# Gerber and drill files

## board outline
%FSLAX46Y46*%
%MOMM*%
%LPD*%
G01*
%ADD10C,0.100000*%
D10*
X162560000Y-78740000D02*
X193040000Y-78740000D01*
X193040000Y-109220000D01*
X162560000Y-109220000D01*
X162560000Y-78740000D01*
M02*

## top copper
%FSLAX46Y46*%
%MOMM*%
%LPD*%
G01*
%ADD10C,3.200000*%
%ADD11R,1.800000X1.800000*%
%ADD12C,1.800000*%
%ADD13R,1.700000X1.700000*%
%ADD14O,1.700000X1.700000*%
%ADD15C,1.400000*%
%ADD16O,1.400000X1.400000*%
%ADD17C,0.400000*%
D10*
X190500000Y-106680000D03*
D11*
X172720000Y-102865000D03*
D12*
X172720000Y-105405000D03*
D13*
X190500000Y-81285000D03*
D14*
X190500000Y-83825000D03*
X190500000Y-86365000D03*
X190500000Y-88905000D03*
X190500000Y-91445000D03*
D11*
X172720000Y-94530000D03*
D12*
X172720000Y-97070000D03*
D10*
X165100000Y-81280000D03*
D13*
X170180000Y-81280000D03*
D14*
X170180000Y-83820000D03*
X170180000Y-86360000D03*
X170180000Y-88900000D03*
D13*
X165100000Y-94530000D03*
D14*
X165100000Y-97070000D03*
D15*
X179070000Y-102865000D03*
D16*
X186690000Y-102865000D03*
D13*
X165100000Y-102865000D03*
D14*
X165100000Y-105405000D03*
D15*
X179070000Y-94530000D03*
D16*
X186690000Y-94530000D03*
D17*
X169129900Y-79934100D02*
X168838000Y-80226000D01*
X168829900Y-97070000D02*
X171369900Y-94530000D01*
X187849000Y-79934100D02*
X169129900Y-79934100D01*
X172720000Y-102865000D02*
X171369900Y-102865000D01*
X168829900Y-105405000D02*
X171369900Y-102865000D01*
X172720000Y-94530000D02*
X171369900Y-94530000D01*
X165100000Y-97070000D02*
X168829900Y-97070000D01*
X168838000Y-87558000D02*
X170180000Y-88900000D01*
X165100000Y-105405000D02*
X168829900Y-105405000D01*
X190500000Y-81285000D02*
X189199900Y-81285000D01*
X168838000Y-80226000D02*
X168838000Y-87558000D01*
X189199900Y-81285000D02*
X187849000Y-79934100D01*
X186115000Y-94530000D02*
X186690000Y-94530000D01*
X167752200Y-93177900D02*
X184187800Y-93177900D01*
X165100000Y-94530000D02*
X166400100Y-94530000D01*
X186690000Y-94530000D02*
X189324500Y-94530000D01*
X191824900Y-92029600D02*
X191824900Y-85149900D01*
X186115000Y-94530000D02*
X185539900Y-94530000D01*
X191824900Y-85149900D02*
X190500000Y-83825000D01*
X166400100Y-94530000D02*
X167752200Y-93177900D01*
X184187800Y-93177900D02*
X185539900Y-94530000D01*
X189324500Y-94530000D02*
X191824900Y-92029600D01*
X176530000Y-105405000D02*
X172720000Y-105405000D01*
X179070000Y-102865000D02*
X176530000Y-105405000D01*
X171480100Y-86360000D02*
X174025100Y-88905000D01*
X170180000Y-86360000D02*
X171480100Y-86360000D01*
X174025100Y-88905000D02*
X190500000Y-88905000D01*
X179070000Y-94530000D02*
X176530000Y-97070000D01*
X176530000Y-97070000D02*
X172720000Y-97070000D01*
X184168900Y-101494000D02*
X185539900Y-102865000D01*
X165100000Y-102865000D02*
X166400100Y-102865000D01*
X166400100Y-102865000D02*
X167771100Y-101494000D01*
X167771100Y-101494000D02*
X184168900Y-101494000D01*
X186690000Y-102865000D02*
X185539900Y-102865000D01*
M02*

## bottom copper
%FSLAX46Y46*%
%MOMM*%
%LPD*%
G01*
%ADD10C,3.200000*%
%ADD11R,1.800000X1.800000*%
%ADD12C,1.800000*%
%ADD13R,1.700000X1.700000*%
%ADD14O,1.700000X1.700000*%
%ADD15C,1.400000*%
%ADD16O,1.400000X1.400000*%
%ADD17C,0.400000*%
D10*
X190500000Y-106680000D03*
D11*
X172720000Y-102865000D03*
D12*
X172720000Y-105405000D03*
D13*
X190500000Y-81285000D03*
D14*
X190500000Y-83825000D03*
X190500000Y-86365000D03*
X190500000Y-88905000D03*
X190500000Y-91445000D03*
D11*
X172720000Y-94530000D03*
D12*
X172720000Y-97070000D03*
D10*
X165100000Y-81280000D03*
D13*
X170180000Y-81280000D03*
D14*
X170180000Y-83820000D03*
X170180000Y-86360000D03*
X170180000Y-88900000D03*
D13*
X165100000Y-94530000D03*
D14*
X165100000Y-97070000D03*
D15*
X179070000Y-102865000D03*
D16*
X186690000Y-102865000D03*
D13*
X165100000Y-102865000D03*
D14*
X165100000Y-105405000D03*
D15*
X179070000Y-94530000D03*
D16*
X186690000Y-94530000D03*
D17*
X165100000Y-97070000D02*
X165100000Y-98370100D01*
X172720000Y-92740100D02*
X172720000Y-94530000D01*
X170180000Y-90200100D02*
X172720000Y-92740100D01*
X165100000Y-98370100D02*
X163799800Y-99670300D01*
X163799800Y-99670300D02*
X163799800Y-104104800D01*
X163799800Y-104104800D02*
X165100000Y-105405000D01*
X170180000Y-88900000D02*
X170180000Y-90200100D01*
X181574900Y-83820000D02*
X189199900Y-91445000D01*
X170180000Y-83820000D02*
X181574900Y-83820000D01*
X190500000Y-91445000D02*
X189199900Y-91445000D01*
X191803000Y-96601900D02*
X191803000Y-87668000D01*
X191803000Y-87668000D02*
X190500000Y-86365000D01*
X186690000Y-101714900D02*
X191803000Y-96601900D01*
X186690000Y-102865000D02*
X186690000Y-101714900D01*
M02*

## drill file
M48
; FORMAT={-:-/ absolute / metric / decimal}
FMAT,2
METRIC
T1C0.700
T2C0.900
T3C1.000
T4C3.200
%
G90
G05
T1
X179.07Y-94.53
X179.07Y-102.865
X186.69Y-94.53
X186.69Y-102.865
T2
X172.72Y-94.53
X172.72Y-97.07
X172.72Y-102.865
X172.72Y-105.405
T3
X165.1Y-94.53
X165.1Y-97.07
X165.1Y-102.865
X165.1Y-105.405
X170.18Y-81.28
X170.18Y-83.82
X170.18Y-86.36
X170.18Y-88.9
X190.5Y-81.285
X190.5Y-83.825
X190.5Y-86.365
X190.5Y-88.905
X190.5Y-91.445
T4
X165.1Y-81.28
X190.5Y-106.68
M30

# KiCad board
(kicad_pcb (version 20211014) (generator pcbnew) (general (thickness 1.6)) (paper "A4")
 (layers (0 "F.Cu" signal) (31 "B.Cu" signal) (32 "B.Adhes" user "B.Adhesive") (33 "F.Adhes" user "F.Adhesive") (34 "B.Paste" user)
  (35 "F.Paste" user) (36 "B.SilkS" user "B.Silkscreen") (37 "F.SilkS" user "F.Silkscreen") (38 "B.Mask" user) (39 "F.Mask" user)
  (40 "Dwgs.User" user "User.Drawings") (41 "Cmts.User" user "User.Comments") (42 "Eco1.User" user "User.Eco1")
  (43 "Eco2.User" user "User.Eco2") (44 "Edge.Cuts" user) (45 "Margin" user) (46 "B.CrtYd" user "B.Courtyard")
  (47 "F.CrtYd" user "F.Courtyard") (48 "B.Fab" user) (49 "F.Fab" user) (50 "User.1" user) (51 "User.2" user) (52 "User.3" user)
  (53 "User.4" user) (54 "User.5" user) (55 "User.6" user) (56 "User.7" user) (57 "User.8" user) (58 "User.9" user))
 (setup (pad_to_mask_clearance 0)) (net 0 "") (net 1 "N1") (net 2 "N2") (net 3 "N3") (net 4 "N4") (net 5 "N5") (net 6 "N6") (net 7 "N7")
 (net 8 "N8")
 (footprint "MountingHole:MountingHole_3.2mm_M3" (layer "F.Cu") (at 190.5 106.68)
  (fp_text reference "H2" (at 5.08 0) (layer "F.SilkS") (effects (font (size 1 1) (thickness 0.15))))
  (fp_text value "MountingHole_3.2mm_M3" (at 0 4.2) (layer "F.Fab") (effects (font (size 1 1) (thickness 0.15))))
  (pad "" thru_hole circle (at 0 0) (size 3.2 3.2) (drill 3.2) (layers *.Cu *.Mask)))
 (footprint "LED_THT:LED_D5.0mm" (layer "F.Cu") (at 172.72 102.865 -90)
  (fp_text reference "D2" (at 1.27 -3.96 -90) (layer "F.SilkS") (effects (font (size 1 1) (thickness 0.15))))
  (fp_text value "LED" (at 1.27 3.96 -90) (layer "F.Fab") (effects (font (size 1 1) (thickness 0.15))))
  (pad "1" thru_hole rect (at 0 0 270) (size 1.8 1.8) (drill 0.9) (layers *.Cu *.Mask) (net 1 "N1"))
  (pad "2" thru_hole circle (at 2.54 0 270) (size 1.8 1.8) (drill 0.9) (layers *.Cu *.Mask) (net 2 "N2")))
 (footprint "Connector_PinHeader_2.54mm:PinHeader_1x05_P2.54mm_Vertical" (layer "F.Cu") (at 190.5 81.285)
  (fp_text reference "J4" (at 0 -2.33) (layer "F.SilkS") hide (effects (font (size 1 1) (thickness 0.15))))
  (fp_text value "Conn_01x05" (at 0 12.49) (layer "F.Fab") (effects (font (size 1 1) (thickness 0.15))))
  (pad "1" thru_hole rect (at 0 0) (size 1.7 1.7) (drill 1) (layers *.Cu *.Mask) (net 1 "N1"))
  (pad "2" thru_hole oval (at 0 2.54) (size 1.7 1.7) (drill 1) (layers *.Cu *.Mask) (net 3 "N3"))
  (pad "3" thru_hole oval (at 0 5.08) (size 1.7 1.7) (drill 1) (layers *.Cu *.Mask) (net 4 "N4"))
  (pad "4" thru_hole oval (at 0 7.62) (size 1.7 1.7) (drill 1) (layers *.Cu *.Mask) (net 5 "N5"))
  (pad "5" thru_hole oval (at 0 10.16) (size 1.7 1.7) (drill 1) (layers *.Cu *.Mask) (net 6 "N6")))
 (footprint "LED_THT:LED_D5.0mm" (layer "F.Cu") (at 172.72 94.53 -90)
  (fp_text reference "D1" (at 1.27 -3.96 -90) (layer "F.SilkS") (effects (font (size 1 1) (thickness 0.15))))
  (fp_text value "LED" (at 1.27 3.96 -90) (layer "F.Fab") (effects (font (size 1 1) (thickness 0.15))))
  (pad "1" thru_hole rect (at 0 0 270) (size 1.8 1.8) (drill 0.9) (layers *.Cu *.Mask) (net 1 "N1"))
  (pad "2" thru_hole circle (at 2.54 0 270) (size 1.8 1.8) (drill 0.9) (layers *.Cu *.Mask) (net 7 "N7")))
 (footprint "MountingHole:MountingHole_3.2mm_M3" (layer "F.Cu") (at 165.1 81.28)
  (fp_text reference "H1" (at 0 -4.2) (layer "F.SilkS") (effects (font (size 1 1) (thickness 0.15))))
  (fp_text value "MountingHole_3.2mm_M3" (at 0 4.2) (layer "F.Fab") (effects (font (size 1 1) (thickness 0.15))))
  (pad "" thru_hole circle (at 0 0) (size 3.2 3.2) (drill 3.2) (layers *.Cu *.Mask)))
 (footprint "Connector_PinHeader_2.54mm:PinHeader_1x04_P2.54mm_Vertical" (layer "F.Cu") (at 170.18 81.28)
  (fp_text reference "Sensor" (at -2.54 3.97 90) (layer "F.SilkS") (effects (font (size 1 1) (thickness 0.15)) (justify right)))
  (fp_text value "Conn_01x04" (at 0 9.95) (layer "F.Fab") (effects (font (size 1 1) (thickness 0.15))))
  (pad "1" thru_hole rect (at 0 0) (size 1.7 1.7) (drill 1) (layers *.Cu *.Mask) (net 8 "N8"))
  (pad "2" thru_hole oval (at 0 2.54) (size 1.7 1.7) (drill 1) (layers *.Cu *.Mask) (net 6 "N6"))
  (pad "3" thru_hole oval (at 0 5.08) (size 1.7 1.7) (drill 1) (layers *.Cu *.Mask) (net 5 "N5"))
  (pad "4" thru_hole oval (at 0 7.62) (size 1.7 1.7) (drill 1) (layers *.Cu *.Mask) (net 1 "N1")))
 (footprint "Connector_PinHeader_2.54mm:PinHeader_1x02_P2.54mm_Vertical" (layer "F.Cu") (at 165.1 94.53)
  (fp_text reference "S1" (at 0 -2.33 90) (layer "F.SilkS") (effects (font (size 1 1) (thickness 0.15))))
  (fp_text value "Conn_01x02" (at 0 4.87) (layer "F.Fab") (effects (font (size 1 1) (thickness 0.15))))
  (pad "1" thru_hole rect (at 0 0) (size 1.7 1.7) (drill 1) (layers *.Cu *.Mask) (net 3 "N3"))
  (pad "2" thru_hole oval (at 0 2.54) (size 1.7 1.7) (drill 1) (layers *.Cu *.Mask) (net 1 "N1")))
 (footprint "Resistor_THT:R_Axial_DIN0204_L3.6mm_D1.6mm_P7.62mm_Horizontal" (layer "F.Cu") (at 179.07 102.865)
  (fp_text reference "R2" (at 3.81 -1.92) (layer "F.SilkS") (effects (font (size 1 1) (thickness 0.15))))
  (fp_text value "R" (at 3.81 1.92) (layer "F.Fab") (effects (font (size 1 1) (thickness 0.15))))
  (pad "1" thru_hole circle (at 0 0) (size 1.4 1.4) (drill 0.7) (layers *.Cu *.Mask) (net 2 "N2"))
  (pad "2" thru_hole oval (at 7.62 0) (size 1.4 1.4) (drill 0.7) (layers *.Cu *.Mask) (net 4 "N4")))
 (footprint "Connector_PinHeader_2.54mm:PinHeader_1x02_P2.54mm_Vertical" (layer "F.Cu") (at 165.1 102.865)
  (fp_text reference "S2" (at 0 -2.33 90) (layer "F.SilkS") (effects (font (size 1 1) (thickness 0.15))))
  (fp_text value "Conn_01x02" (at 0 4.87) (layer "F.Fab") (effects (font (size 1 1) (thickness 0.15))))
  (pad "1" thru_hole rect (at 0 0) (size 1.7 1.7) (drill 1) (layers *.Cu *.Mask) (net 4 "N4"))
  (pad "2" thru_hole oval (at 0 2.54) (size 1.7 1.7) (drill 1) (layers *.Cu *.Mask) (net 1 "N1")))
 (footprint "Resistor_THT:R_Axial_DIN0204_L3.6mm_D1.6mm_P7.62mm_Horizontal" (layer "F.Cu") (at 179.07 94.53)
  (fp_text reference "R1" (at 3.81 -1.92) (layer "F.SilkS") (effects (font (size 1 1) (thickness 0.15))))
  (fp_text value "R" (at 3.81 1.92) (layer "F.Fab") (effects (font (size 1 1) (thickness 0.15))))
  (pad "1" thru_hole circle (at 0 0) (size 1.4 1.4) (drill 0.7) (layers *.Cu *.Mask) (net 7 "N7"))
  (pad "2" thru_hole oval (at 7.62 0) (size 1.4 1.4) (drill 0.7) (layers *.Cu *.Mask) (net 3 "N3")))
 (gr_rect (start 162.56 78.74) (end 193.04 109.22) (layer "Edge.Cuts") (width 0.1) (fill none))
 (segment (start 169.1299 79.9341) (end 168.838 80.226) (width 0.4) (layer "F.Cu") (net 1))
 (segment (start 168.8299 97.07) (end 171.3699 94.53) (width 0.4) (layer "F.Cu") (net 1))
 (segment (start 187.849 79.9341) (end 169.1299 79.9341) (width 0.4) (layer "F.Cu") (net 1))
 (segment (start 172.72 102.865) (end 171.3699 102.865) (width 0.4) (layer "F.Cu") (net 1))
 (segment (start 168.8299 105.405) (end 171.3699 102.865) (width 0.4) (layer "F.Cu") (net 1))
 (segment (start 172.72 94.53) (end 171.3699 94.53) (width 0.4) (layer "F.Cu") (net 1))
 (segment (start 165.1 97.07) (end 168.8299 97.07) (width 0.4) (layer "F.Cu") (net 1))
 (segment (start 168.838 87.558) (end 170.18 88.9) (width 0.4) (layer "F.Cu") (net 1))
 (segment (start 165.1 105.405) (end 168.8299 105.405) (width 0.4) (layer "F.Cu") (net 1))
 (segment (start 190.5 81.285) (end 189.1999 81.285) (width 0.4) (layer "F.Cu") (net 1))
 (segment (start 168.838 80.226) (end 168.838 87.558) (width 0.4) (layer "F.Cu") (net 1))
 (segment (start 189.1999 81.285) (end 187.849 79.9341) (width 0.4) (layer "F.Cu") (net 1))
 (segment (start 165.1 97.07) (end 165.1 98.3701) (width 0.4) (layer "B.Cu") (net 1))
 (segment (start 172.72 92.7401) (end 172.72 94.53) (width 0.4) (layer "B.Cu") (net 1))
 (segment (start 170.18 90.2001) (end 172.72 92.7401) (width 0.4) (layer "B.Cu") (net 1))
 (segment (start 165.1 98.3701) (end 163.7998 99.6703) (width 0.4) (layer "B.Cu") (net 1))
 (segment (start 163.7998 99.6703) (end 163.7998 104.1048) (width 0.4) (layer "B.Cu") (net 1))
 (segment (start 163.7998 104.1048) (end 165.1 105.405) (width 0.4) (layer "B.Cu") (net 1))
 (segment (start 170.18 88.9) (end 170.18 90.2001) (width 0.4) (layer "B.Cu") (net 1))
 (segment (start 186.115 94.53) (end 186.69 94.53) (width 0.4) (layer "F.Cu") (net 3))
 (segment (start 167.7522 93.1779) (end 184.1878 93.1779) (width 0.4) (layer "F.Cu") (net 3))
 (segment (start 165.1 94.53) (end 166.4001 94.53) (width 0.4) (layer "F.Cu") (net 3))
 (segment (start 186.69 94.53) (end 189.3245 94.53) (width 0.4) (layer "F.Cu") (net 3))
 (segment (start 191.8249 92.0296) (end 191.8249 85.1499) (width 0.4) (layer "F.Cu") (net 3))
 (segment (start 186.115 94.53) (end 185.5399 94.53) (width 0.4) (layer "F.Cu") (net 3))
 (segment (start 191.8249 85.1499) (end 190.5 83.825) (width 0.4) (layer "F.Cu") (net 3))
 (segment (start 166.4001 94.53) (end 167.7522 93.1779) (width 0.4) (layer "F.Cu") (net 3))
 (segment (start 184.1878 93.1779) (end 185.5399 94.53) (width 0.4) (layer "F.Cu") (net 3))
 (segment (start 189.3245 94.53) (end 191.8249 92.0296) (width 0.4) (layer "F.Cu") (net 3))
 (segment (start 176.53 105.405) (end 172.72 105.405) (width 0.4) (layer "F.Cu") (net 2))
 (segment (start 179.07 102.865) (end 176.53 105.405) (width 0.4) (layer "F.Cu") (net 2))
 (segment (start 181.5749 83.82) (end 189.1999 91.445) (width 0.4) (layer "B.Cu") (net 6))
 (segment (start 170.18 83.82) (end 181.5749 83.82) (width 0.4) (layer "B.Cu") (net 6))
 (segment (start 190.5 91.445) (end 189.1999 91.445) (width 0.4) (layer "B.Cu") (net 6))
 (segment (start 171.4801 86.36) (end 174.0251 88.905) (width 0.4) (layer "F.Cu") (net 5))
 (segment (start 170.18 86.36) (end 171.4801 86.36) (width 0.4) (layer "F.Cu") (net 5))
 (segment (start 174.0251 88.905) (end 190.5 88.905) (width 0.4) (layer "F.Cu") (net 5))
 (segment (start 179.07 94.53) (end 176.53 97.07) (width 0.4) (layer "F.Cu") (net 7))
 (segment (start 176.53 97.07) (end 172.72 97.07) (width 0.4) (layer "F.Cu") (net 7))
 (segment (start 184.1689 101.494) (end 185.5399 102.865) (width 0.4) (layer "F.Cu") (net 4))
 (segment (start 165.1 102.865) (end 166.4001 102.865) (width 0.4) (layer "F.Cu") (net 4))
 (segment (start 166.4001 102.865) (end 167.7711 101.494) (width 0.4) (layer "F.Cu") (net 4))
 (segment (start 167.7711 101.494) (end 184.1689 101.494) (width 0.4) (layer "F.Cu") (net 4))
 (segment (start 186.69 102.865) (end 185.5399 102.865) (width 0.4) (layer "F.Cu") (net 4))
 (segment (start 191.803 96.6019) (end 191.803 87.668) (width 0.4) (layer "B.Cu") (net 4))
 (segment (start 191.803 87.668) (end 190.5 86.365) (width 0.4) (layer "B.Cu") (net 4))
 (segment (start 186.69 101.7149) (end 191.803 96.6019) (width 0.4) (layer "B.Cu") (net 4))
 (segment (start 186.69 102.865) (end 186.69 101.7149) (width 0.4) (layer "B.Cu") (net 4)))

